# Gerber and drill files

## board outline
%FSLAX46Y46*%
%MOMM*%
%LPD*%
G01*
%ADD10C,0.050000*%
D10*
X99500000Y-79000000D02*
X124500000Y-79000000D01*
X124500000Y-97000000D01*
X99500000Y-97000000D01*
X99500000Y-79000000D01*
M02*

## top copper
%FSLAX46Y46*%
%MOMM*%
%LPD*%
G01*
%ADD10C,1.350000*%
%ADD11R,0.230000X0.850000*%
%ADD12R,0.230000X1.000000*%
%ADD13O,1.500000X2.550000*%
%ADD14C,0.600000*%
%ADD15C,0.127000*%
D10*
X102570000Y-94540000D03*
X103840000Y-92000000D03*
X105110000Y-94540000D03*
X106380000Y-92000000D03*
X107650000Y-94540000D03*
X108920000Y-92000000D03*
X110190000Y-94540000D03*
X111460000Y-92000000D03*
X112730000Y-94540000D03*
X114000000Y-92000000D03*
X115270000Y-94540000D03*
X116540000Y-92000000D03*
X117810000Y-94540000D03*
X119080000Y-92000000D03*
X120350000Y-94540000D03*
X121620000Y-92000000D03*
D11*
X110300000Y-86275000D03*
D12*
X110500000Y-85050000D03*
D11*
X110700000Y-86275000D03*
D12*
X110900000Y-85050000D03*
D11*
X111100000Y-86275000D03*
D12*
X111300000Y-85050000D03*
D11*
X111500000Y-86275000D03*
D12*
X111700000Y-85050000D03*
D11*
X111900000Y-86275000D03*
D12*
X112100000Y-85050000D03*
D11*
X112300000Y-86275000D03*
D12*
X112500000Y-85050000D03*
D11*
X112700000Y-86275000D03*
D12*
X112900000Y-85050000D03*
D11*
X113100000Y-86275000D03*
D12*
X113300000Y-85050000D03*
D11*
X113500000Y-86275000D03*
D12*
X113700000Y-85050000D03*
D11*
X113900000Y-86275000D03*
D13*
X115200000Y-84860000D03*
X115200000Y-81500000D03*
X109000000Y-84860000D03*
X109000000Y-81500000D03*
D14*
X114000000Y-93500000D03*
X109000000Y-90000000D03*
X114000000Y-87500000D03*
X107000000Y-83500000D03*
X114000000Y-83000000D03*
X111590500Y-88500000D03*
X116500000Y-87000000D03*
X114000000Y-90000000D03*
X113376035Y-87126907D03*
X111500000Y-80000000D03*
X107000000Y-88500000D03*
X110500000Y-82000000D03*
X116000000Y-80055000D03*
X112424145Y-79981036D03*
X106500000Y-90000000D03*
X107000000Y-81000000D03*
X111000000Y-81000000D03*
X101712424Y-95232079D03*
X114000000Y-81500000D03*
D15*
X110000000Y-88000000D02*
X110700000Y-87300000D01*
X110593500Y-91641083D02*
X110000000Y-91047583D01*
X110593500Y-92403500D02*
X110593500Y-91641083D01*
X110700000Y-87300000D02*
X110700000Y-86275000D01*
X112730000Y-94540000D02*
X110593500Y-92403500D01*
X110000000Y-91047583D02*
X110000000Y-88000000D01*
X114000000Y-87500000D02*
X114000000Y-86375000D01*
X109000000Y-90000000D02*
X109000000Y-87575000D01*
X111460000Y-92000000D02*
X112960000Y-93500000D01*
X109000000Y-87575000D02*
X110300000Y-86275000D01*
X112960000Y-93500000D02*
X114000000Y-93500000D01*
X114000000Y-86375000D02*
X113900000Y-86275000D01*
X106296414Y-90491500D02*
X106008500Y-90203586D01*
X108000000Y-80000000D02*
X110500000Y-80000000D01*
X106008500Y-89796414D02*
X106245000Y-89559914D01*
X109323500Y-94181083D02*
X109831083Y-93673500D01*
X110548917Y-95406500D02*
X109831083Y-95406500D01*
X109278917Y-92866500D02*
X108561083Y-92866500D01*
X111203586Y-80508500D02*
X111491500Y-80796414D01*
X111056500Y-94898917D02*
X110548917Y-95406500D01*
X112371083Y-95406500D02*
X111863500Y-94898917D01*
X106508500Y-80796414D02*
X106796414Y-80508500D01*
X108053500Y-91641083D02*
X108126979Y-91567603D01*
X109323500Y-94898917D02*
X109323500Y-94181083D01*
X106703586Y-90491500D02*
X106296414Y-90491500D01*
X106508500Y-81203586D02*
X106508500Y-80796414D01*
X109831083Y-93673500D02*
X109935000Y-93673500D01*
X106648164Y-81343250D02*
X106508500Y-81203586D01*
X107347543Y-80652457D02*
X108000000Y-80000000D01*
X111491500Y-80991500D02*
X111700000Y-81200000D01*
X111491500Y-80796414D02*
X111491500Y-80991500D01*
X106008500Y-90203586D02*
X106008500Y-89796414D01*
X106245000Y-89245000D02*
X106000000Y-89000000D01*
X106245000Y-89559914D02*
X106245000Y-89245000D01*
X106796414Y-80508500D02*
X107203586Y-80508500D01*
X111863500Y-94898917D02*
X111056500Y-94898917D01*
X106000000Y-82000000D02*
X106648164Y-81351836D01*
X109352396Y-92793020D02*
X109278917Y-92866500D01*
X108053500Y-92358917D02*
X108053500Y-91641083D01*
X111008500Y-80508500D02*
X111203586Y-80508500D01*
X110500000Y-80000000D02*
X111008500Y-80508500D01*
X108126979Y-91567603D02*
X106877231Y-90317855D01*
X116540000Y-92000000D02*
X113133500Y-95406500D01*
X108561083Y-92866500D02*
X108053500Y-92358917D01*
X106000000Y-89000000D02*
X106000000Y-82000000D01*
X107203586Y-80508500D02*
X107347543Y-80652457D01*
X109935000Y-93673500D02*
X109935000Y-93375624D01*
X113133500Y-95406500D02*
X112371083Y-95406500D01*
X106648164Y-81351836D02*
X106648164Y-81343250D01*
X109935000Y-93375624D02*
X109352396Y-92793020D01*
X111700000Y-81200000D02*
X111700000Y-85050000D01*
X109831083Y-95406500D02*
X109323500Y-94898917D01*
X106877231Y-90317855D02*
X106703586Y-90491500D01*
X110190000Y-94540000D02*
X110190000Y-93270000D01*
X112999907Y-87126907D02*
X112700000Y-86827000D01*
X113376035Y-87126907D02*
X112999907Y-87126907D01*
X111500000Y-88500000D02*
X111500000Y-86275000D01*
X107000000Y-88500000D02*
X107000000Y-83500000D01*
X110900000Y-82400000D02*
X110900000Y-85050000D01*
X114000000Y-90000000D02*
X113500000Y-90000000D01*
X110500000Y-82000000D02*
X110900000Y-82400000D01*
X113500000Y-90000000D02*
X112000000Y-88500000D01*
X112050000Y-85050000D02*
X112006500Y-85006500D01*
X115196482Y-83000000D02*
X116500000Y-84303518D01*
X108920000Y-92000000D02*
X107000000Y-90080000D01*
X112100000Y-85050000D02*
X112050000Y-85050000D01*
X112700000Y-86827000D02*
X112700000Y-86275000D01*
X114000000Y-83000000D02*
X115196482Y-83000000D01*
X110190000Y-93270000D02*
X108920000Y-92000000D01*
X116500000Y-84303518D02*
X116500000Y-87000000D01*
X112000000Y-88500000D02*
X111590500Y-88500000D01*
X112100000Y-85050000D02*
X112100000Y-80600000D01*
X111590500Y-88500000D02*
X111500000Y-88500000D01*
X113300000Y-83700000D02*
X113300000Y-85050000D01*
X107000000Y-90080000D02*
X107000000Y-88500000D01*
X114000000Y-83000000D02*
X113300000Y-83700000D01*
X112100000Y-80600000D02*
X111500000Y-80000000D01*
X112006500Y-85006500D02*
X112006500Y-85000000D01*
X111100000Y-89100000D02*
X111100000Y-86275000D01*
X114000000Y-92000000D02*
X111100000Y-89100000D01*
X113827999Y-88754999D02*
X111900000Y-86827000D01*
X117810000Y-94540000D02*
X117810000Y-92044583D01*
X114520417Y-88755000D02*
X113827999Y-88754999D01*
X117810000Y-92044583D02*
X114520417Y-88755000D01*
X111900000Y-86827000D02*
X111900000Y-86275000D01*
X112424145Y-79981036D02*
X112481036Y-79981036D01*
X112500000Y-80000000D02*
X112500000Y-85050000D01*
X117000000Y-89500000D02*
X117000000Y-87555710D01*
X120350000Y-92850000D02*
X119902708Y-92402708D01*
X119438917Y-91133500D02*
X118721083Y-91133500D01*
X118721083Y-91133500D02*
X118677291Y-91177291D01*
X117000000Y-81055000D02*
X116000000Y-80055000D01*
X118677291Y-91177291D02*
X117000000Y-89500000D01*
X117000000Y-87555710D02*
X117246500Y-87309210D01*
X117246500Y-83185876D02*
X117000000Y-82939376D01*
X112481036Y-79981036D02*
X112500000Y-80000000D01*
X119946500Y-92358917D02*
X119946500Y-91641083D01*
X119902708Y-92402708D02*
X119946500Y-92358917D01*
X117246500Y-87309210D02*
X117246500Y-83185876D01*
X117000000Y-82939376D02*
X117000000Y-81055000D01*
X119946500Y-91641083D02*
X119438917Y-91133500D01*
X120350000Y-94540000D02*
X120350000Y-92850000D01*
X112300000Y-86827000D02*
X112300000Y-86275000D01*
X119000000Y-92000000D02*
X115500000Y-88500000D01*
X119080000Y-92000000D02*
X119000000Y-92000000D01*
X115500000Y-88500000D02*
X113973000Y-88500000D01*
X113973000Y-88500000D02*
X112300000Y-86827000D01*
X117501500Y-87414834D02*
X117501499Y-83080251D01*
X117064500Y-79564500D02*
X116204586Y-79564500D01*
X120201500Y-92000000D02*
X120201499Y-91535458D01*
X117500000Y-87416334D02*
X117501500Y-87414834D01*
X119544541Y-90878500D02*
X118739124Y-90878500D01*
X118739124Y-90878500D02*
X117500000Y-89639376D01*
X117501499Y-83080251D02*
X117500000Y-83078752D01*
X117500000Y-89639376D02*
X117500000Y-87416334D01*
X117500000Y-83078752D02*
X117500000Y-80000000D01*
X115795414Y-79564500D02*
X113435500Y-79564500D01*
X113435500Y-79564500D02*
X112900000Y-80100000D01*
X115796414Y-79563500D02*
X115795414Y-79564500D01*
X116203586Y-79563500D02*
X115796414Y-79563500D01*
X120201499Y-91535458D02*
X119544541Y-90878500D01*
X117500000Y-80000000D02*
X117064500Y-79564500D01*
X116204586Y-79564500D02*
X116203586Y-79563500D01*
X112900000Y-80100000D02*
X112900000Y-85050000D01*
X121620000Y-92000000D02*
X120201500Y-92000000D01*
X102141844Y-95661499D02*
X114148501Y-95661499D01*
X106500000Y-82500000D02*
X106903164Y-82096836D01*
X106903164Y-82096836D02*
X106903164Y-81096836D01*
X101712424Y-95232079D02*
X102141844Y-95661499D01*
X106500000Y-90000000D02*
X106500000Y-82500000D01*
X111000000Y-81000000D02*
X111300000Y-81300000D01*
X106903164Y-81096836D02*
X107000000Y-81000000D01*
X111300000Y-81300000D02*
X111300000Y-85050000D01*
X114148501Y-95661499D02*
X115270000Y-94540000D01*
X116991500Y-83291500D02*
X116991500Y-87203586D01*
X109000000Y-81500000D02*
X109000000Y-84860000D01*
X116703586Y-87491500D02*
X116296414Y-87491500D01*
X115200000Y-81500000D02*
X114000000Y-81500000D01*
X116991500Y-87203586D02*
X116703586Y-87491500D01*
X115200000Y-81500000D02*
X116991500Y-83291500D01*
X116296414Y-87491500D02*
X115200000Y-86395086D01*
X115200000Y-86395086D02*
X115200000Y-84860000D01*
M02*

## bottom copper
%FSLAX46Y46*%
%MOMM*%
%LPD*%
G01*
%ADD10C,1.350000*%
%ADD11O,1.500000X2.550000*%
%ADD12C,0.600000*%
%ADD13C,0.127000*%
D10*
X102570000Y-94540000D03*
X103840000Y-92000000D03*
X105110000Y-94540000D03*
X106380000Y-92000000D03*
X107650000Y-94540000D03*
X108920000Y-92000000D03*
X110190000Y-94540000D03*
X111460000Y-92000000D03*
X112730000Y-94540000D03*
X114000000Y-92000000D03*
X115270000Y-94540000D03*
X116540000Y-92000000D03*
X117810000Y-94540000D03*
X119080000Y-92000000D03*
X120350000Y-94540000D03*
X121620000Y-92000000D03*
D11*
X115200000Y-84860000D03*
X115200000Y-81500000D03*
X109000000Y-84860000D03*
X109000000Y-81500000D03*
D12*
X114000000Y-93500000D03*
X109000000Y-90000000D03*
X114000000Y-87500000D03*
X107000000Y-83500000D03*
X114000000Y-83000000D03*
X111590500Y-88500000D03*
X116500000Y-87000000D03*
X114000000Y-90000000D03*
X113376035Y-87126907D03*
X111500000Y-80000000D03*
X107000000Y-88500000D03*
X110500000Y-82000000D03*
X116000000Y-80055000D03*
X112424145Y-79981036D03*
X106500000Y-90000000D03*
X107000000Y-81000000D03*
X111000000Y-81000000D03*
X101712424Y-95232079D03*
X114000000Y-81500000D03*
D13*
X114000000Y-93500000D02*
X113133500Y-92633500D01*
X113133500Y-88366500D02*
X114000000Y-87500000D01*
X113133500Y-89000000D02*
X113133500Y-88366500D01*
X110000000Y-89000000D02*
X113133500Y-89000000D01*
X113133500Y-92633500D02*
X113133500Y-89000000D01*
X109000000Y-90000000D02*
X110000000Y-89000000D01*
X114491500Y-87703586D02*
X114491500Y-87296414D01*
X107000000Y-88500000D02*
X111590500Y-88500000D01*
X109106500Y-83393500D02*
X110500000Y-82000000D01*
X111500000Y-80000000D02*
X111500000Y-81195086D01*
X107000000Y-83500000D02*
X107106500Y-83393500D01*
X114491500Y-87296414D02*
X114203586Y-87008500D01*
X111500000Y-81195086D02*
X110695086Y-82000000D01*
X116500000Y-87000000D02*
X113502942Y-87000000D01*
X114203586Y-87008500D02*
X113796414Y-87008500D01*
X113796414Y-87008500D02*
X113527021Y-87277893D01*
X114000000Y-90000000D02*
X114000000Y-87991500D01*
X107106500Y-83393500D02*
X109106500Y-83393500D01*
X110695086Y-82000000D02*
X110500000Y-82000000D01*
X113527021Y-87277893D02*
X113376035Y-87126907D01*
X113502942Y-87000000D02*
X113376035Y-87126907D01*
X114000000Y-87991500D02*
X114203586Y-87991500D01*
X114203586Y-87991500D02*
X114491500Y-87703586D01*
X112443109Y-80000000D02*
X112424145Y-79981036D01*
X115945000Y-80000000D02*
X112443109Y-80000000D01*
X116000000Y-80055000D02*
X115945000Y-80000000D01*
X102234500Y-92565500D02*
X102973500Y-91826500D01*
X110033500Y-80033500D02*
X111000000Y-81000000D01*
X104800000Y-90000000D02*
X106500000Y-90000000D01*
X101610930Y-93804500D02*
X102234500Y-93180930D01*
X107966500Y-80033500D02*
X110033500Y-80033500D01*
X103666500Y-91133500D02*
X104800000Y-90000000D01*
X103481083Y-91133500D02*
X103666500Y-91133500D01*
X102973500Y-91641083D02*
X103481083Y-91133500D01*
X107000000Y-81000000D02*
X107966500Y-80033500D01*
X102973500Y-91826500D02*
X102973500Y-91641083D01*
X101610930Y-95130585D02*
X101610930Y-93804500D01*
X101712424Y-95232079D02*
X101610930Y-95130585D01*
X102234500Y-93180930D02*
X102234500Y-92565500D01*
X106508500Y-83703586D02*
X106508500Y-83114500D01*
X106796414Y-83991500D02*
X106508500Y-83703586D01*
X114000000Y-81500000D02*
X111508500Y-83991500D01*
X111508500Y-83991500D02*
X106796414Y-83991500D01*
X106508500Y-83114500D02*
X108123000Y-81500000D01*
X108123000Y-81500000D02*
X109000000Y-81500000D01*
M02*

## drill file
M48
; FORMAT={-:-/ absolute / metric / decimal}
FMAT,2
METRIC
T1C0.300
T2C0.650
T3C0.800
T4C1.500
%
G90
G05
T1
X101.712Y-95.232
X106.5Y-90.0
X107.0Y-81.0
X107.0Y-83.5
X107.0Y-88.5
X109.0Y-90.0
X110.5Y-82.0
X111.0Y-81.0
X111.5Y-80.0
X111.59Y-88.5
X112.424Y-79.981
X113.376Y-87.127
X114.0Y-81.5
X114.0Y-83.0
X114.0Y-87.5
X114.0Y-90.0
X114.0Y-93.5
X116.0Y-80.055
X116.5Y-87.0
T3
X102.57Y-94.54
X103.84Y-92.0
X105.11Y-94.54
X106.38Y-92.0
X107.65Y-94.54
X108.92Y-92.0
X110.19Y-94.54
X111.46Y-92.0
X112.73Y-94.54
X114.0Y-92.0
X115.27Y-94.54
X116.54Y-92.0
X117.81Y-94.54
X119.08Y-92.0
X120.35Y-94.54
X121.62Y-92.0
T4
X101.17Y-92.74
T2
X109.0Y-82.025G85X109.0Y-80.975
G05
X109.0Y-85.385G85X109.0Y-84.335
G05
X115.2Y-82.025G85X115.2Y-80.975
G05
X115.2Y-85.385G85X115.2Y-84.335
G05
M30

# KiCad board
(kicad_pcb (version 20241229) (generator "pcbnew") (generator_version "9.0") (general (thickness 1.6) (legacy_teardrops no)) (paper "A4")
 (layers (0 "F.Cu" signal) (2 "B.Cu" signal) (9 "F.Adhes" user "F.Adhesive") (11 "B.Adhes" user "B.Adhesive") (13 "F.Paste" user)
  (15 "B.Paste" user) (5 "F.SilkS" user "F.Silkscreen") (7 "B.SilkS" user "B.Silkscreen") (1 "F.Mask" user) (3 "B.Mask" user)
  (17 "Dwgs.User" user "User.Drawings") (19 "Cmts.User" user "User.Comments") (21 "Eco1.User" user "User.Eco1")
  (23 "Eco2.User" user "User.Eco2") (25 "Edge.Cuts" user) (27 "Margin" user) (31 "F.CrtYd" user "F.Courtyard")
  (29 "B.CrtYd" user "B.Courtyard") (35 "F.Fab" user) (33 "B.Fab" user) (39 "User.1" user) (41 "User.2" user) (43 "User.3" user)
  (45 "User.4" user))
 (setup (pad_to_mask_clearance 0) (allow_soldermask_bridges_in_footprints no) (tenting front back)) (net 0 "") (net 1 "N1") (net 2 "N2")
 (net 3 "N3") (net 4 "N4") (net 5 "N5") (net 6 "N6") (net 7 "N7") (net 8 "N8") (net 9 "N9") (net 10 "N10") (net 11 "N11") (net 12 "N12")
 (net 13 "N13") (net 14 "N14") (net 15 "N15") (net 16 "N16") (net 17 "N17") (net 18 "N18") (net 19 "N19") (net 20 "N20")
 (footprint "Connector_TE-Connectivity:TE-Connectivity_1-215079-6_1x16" (layer "F.Cu") (at 111.46 93.27)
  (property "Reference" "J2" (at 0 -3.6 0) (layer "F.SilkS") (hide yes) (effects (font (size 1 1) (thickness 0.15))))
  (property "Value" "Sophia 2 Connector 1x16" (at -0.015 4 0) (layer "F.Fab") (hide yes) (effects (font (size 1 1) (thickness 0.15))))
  (pad "" np_thru_hole circle (at -10.29 -0.53) (size 1.5 1.5) (drill 1.5) (layers "*.Cu" "*.Mask"))
  (pad "1" thru_hole circle (at -8.89 1.27) (size 1.35 1.35) (drill 0.8) (layers "*.Cu" "*.Mask") (remove_unused_layers no) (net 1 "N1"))
  (pad "2" thru_hole circle (at -7.62 -1.27) (size 1.35 1.35) (drill 0.8) (layers "*.Cu" "*.Mask") (remove_unused_layers no) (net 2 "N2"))
  (pad "3" thru_hole circle (at -6.35 1.27) (size 1.35 1.35) (drill 0.8) (layers "*.Cu" "*.Mask") (remove_unused_layers no) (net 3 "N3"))
  (pad "4" thru_hole circle (at -5.08 -1.27) (size 1.35 1.35) (drill 0.8) (layers "*.Cu" "*.Mask") (remove_unused_layers no) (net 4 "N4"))
  (pad "5" thru_hole circle (at -3.81 1.27) (size 1.35 1.35) (drill 0.8) (layers "*.Cu" "*.Mask") (remove_unused_layers no) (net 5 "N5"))
  (pad "6" thru_hole circle (at -2.54 -1.27) (size 1.35 1.35) (drill 0.8) (layers "*.Cu" "*.Mask") (remove_unused_layers no) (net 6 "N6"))
  (pad "7" thru_hole circle (at -1.27 1.27) (size 1.35 1.35) (drill 0.8) (layers "*.Cu" "*.Mask") (remove_unused_layers no) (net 6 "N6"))
  (pad "8" thru_hole circle (at 0 -1.27) (size 1.35 1.35) (drill 0.8) (layers "*.Cu" "*.Mask") (remove_unused_layers no) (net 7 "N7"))
  (pad "9" thru_hole circle (at 1.27 1.27) (size 1.35 1.35) (drill 0.8) (layers "*.Cu" "*.Mask") (remove_unused_layers no) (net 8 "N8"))
  (pad "10" thru_hole circle (at 2.54 -1.27) (size 1.35 1.35) (drill 0.8) (layers "*.Cu" "*.Mask") (remove_unused_layers no) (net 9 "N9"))
  (pad "11" thru_hole circle (at 3.81 1.27) (size 1.35 1.35) (drill 0.8) (layers "*.Cu" "*.Mask") (remove_unused_layers no) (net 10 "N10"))
  (pad "12" thru_hole circle (at 5.08 -1.27) (size 1.35 1.35) (drill 0.8) (layers "*.Cu" "*.Mask") (remove_unused_layers no) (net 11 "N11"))
  (pad "13" thru_hole circle (at 6.35 1.27) (size 1.35 1.35) (drill 0.8) (layers "*.Cu" "*.Mask") (remove_unused_layers no) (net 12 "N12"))
  (pad "14" thru_hole circle (at 7.62 -1.27) (size 1.35 1.35) (drill 0.8) (layers "*.Cu" "*.Mask") (remove_unused_layers no) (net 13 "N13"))
  (pad "15" thru_hole circle (at 8.89 1.27) (size 1.35 1.35) (drill 0.8) (layers "*.Cu" "*.Mask") (remove_unused_layers no) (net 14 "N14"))
  (pad "16" thru_hole circle (at 10.16 -1.27) (size 1.35 1.35) (drill 0.8) (layers "*.Cu" "*.Mask") (remove_unused_layers no) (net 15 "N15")))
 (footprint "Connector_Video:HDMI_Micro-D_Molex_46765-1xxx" (layer "F.Cu") (at 112.1 81.5 180)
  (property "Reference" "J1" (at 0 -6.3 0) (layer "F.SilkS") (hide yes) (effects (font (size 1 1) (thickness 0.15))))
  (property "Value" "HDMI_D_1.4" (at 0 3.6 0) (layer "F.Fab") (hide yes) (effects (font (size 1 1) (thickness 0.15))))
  (pad "1" smd rect (at 1.8 -4.775 180) (size 0.23 0.85) (layers "F.Cu" "F.Mask" "F.Paste") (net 7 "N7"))
  (pad "2" smd rect (at 1.6 -3.55 180) (size 0.23 1) (layers "F.Cu" "F.Mask" "F.Paste") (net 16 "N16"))
  (pad "3" smd rect (at 1.4 -4.775 180) (size 0.23 0.85) (layers "F.Cu" "F.Mask" "F.Paste") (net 8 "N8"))
  (pad "4" smd rect (at 1.2 -3.55 180) (size 0.23 1) (layers "F.Cu" "F.Mask" "F.Paste") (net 6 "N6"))
  (pad "5" smd rect (at 1 -4.775 180) (size 0.23 0.85) (layers "F.Cu" "F.Mask" "F.Paste") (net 9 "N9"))
  (pad "6" smd rect (at 0.8 -3.55 180) (size 0.23 1) (layers "F.Cu" "F.Mask" "F.Paste") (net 10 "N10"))
  (pad "7" smd rect (at 0.6 -4.775 180) (size 0.23 0.85) (layers "F.Cu" "F.Mask" "F.Paste") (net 6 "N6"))
  (pad "8" smd rect (at 0.4 -3.55 180) (size 0.23 1) (layers "F.Cu" "F.Mask" "F.Paste") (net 11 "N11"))
  (pad "9" smd rect (at 0.2 -4.775 180) (size 0.23 0.85) (layers "F.Cu" "F.Mask" "F.Paste") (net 12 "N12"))
  (pad "10" smd rect (at 0 -3.55 180) (size 0.23 1) (layers "F.Cu" "F.Mask" "F.Paste") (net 6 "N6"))
  (pad "11" smd rect (at -0.2 -4.775 180) (size 0.23 0.85) (layers "F.Cu" "F.Mask" "F.Paste") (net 13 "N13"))
  (pad "12" smd rect (at -0.4 -3.55 180) (size 0.23 1) (layers "F.Cu" "F.Mask" "F.Paste") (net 14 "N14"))
  (pad "13" smd rect (at -0.6 -4.775 180) (size 0.23 0.85) (layers "F.Cu" "F.Mask" "F.Paste") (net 6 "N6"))
  (pad "14" smd rect (at -0.8 -3.55 180) (size 0.23 1) (layers "F.Cu" "F.Mask" "F.Paste") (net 15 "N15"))
  (pad "15" smd rect (at -1 -4.775 180) (size 0.23 0.85) (layers "F.Cu" "F.Mask" "F.Paste") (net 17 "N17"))
  (pad "16" smd rect (at -1.2 -3.55 180) (size 0.23 1) (layers "F.Cu" "F.Mask" "F.Paste") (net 6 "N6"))
  (pad "17" smd rect (at -1.4 -4.775 180) (size 0.23 0.85) (layers "F.Cu" "F.Mask" "F.Paste") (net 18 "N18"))
  (pad "18" smd rect (at -1.6 -3.55 180) (size 0.23 1) (layers "F.Cu" "F.Mask" "F.Paste") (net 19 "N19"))
  (pad "19" smd rect (at -1.8 -4.775 180) (size 0.23 0.85) (layers "F.Cu" "F.Mask" "F.Paste") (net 7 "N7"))
  (pad "SH" thru_hole oval (at -3.1 -3.36 180) (size 1.5 2.55) (drill oval 0.65 1.7) (layers "*.Cu" "*.Mask") (remove_unused_layers no)
   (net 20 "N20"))
  (pad "SH" thru_hole oval (at -3.1 0 180) (size 1.5 2.55) (drill oval 0.65 1.7) (layers "*.Cu" "*.Mask") (remove_unused_layers no)
   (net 20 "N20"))
  (pad "SH" thru_hole oval (at 3.1 -3.36 180) (size 1.5 2.55) (drill oval 0.65 1.7) (layers "*.Cu" "*.Mask") (remove_unused_layers no)
   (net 20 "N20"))
  (pad "SH" thru_hole oval (at 3.1 0 180) (size 1.5 2.55) (drill oval 0.65 1.7) (layers "*.Cu" "*.Mask") (remove_unused_layers no)
   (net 20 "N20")))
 (gr_rect (start 99.5 79) (end 124.5 97) (stroke (width 0.05) (type default)) (fill no) (layer "Edge.Cuts"))
 (segment (start 110 88) (end 110.7 87.3) (width 0.127) (layer "F.Cu") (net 8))
 (segment (start 110.5935 91.641083) (end 110 91.047583) (width 0.127) (layer "F.Cu") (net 8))
 (segment (start 110.5935 92.4035) (end 110.5935 91.641083) (width 0.127) (layer "F.Cu") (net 8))
 (segment (start 110.7 87.3) (end 110.7 86.275) (width 0.127) (layer "F.Cu") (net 8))
 (segment (start 112.73 94.54) (end 110.5935 92.4035) (width 0.127) (layer "F.Cu") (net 8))
 (segment (start 110 91.047583) (end 110 88) (width 0.127) (layer "F.Cu") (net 8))
 (segment (start 114 87.5) (end 114 86.375) (width 0.127) (layer "F.Cu") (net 7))
 (segment (start 109 90) (end 109 87.575) (width 0.127) (layer "F.Cu") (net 7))
 (segment (start 111.46 92) (end 112.96 93.5) (width 0.127) (layer "F.Cu") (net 7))
 (segment (start 109 87.575) (end 110.3 86.275) (width 0.127) (layer "F.Cu") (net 7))
 (segment (start 112.96 93.5) (end 114 93.5) (width 0.127) (layer "F.Cu") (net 7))
 (segment (start 114 86.375) (end 113.9 86.275) (width 0.127) (layer "F.Cu") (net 7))
 (via (at 114 93.5) (size 0.6) (drill 0.3) (layers "F.Cu" "B.Cu") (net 7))
 (via (at 109 90) (size 0.6) (drill 0.3) (layers "F.Cu" "B.Cu") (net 7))
 (via (at 114 87.5) (size 0.6) (drill 0.3) (layers "F.Cu" "B.Cu") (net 7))
 (segment (start 114 93.5) (end 113.1335 92.6335) (width 0.127) (layer "B.Cu") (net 7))
 (segment (start 113.1335 88.3665) (end 114 87.5) (width 0.127) (layer "B.Cu") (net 7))
 (segment (start 113.1335 89) (end 113.1335 88.3665) (width 0.127) (layer "B.Cu") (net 7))
 (segment (start 110 89) (end 113.1335 89) (width 0.127) (layer "B.Cu") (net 7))
 (segment (start 113.1335 92.6335) (end 113.1335 89) (width 0.127) (layer "B.Cu") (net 7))
 (segment (start 109 90) (end 110 89) (width 0.127) (layer "B.Cu") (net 7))
 (segment (start 106.296414 90.4915) (end 106.0085 90.203586) (width 0.127) (layer "F.Cu") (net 11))
 (segment (start 108 80) (end 110.5 80) (width 0.127) (layer "F.Cu") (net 11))
 (segment (start 106.0085 89.796414) (end 106.245 89.559914) (width 0.127) (layer "F.Cu") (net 11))
 (segment (start 109.3235 94.181083) (end 109.831083 93.6735) (width 0.127) (layer "F.Cu") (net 11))
 (segment (start 110.548917 95.4065) (end 109.831083 95.4065) (width 0.127) (layer "F.Cu") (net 11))
 (segment (start 109.278917 92.8665) (end 108.561083 92.8665) (width 0.127) (layer "F.Cu") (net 11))
 (segment (start 111.203586 80.5085) (end 111.4915 80.796414) (width 0.127) (layer "F.Cu") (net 11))
 (segment (start 111.0565 94.898917) (end 110.548917 95.4065) (width 0.127) (layer "F.Cu") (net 11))
 (segment (start 112.371083 95.4065) (end 111.8635 94.898917) (width 0.127) (layer "F.Cu") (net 11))
 (segment (start 106.5085 80.796414) (end 106.796414 80.5085) (width 0.127) (layer "F.Cu") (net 11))
 (segment (start 108.0535 91.641083) (end 108.126979 91.567603) (width 0.127) (layer "F.Cu") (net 11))
 (segment (start 109.3235 94.898917) (end 109.3235 94.181083) (width 0.127) (layer "F.Cu") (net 11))
 (segment (start 106.703586 90.4915) (end 106.296414 90.4915) (width 0.127) (layer "F.Cu") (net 11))
 (segment (start 106.5085 81.203586) (end 106.5085 80.796414) (width 0.127) (layer "F.Cu") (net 11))
 (segment (start 109.831083 93.6735) (end 109.935 93.6735) (width 0.127) (layer "F.Cu") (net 11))
 (segment (start 106.648164 81.34325) (end 106.5085 81.203586) (width 0.127) (layer "F.Cu") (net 11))
 (segment (start 107.347543 80.652457) (end 108 80) (width 0.127) (layer "F.Cu") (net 11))
 (segment (start 111.4915 80.9915) (end 111.7 81.2) (width 0.127) (layer "F.Cu") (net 11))
 (segment (start 111.4915 80.796414) (end 111.4915 80.9915) (width 0.127) (layer "F.Cu") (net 11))
 (segment (start 106.0085 90.203586) (end 106.0085 89.796414) (width 0.127) (layer "F.Cu") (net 11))
 (segment (start 106.245 89.245) (end 106 89) (width 0.127) (layer "F.Cu") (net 11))
 (segment (start 106.245 89.559914) (end 106.245 89.245) (width 0.127) (layer "F.Cu") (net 11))
 (segment (start 106.796414 80.5085) (end 107.203586 80.5085) (width 0.127) (layer "F.Cu") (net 11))
 (segment (start 111.8635 94.898917) (end 111.0565 94.898917) (width 0.127) (layer "F.Cu") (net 11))
 (segment (start 106 82) (end 106.648164 81.351836) (width 0.127) (layer "F.Cu") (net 11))
 (segment (start 109.352396 92.79302) (end 109.278917 92.8665) (width 0.127) (layer "F.Cu") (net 11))
 (segment (start 108.0535 92.358917) (end 108.0535 91.641083) (width 0.127) (layer "F.Cu") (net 11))
 (segment (start 111.0085 80.5085) (end 111.203586 80.5085) (width 0.127) (layer "F.Cu") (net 11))
 (segment (start 110.5 80) (end 111.0085 80.5085) (width 0.127) (layer "F.Cu") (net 11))
 (segment (start 108.126979 91.567603) (end 106.877231 90.317855) (width 0.127) (layer "F.Cu") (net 11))
 (segment (start 116.54 92) (end 113.1335 95.4065) (width 0.127) (layer "F.Cu") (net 11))
 (segment (start 108.561083 92.8665) (end 108.0535 92.358917) (width 0.127) (layer "F.Cu") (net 11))
 (segment (start 106 89) (end 106 82) (width 0.127) (layer "F.Cu") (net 11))
 (segment (start 107.203586 80.5085) (end 107.347543 80.652457) (width 0.127) (layer "F.Cu") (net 11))
 (segment (start 109.935 93.6735) (end 109.935 93.375624) (width 0.127) (layer "F.Cu") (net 11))
 (segment (start 113.1335 95.4065) (end 112.371083 95.4065) (width 0.127) (layer "F.Cu") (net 11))
 (segment (start 106.648164 81.351836) (end 106.648164 81.34325) (width 0.127) (layer "F.Cu") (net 11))
 (segment (start 109.935 93.375624) (end 109.352396 92.79302) (width 0.127) (layer "F.Cu") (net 11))
 (segment (start 111.7 81.2) (end 111.7 85.05) (width 0.127) (layer "F.Cu") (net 11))
 (segment (start 109.831083 95.4065) (end 109.3235 94.898917) (width 0.127) (layer "F.Cu") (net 11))
 (segment (start 106.877231 90.317855) (end 106.703586 90.4915) (width 0.127) (layer "F.Cu") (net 11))
 (segment (start 110.19 94.54) (end 110.19 93.27) (width 0.127) (layer "F.Cu") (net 6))
 (segment (start 112.999907 87.126907) (end 112.7 86.827) (width 0.127) (layer "F.Cu") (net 6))
 (segment (start 113.376035 87.126907) (end 112.999907 87.126907) (width 0.127) (layer "F.Cu") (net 6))
 (segment (start 111.5 88.5) (end 111.5 86.275) (width 0.127) (layer "F.Cu") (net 6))
 (segment (start 107 88.5) (end 107 83.5) (width 0.127) (layer "F.Cu") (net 6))
 (segment (start 110.9 82.4) (end 110.9 85.05) (width 0.127) (layer "F.Cu") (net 6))
 (segment (start 114 90) (end 113.5 90) (width 0.127) (layer "F.Cu") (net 6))
 (segment (start 110.5 82) (end 110.9 82.4) (width 0.127) (layer "F.Cu") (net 6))
 (segment (start 113.5 90) (end 112 88.5) (width 0.127) (layer "F.Cu") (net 6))
 (segment (start 112.05 85.05) (end 112.0065 85.0065) (width 0.127) (layer "F.Cu") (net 6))
 (segment (start 115.196482 83) (end 116.5 84.303518) (width 0.127) (layer "F.Cu") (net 6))
 (segment (start 108.92 92) (end 107 90.08) (width 0.127) (layer "F.Cu") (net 6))
 (segment (start 112.1 85.05) (end 112.05 85.05) (width 0.127) (layer "F.Cu") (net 6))
 (segment (start 112.7 86.827) (end 112.7 86.275) (width 0.127) (layer "F.Cu") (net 6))
 (segment (start 114 83) (end 115.196482 83) (width 0.127) (layer "F.Cu") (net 6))
 (segment (start 110.19 93.27) (end 108.92 92) (width 0.127) (layer "F.Cu") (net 6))
 (segment (start 116.5 84.303518) (end 116.5 87) (width 0.127) (layer "F.Cu") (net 6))
 (segment (start 112 88.5) (end 111.5905 88.5) (width 0.127) (layer "F.Cu") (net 6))
 (segment (start 112.1 85.05) (end 112.1 80.6) (width 0.127) (layer "F.Cu") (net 6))
 (segment (start 111.5905 88.5) (end 111.5 88.5) (width 0.127) (layer "F.Cu") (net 6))
 (segment (start 113.3 83.7) (end 113.3 85.05) (width 0.127) (layer "F.Cu") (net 6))
 (segment (start 107 90.08) (end 107 88.5) (width 0.127) (layer "F.Cu") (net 6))
 (segment (start 114 83) (end 113.3 83.7) (width 0.127) (layer "F.Cu") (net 6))
 (segment (start 112.1 80.6) (end 111.5 80) (width 0.127) (layer "F.Cu") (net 6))
 (segment (start 112.0065 85.0065) (end 112.0065 85) (width 0.127) (layer "F.Cu") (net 6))
 (via (at 107 83.5) (size 0.6) (drill 0.3) (layers "F.Cu" "B.Cu") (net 6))
 (via (at 114 83) (size 0.6) (drill 0.3) (layers "F.Cu" "B.Cu") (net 6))
 (via (at 111.5905 88.5) (size 0.6) (drill 0.3) (layers "F.Cu" "B.Cu") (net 6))
 (via (at 116.5 87) (size 0.6) (drill 0.3) (layers "F.Cu" "B.Cu") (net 6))
 (via (at 114 90) (size 0.6) (drill 0.3) (layers "F.Cu" "B.Cu") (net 6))
 (via (at 113.376035 87.126907) (size 0.6) (drill 0.3) (layers "F.Cu" "B.Cu") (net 6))
 (via (at 111.5 80) (size 0.6) (drill 0.3) (layers "F.Cu" "B.Cu") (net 6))
 (via (at 107 88.5) (size 0.6) (drill 0.3) (layers "F.Cu" "B.Cu") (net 6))
 (via (at 110.5 82) (size 0.6) (drill 0.3) (layers "F.Cu" "B.Cu") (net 6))
 (segment (start 114.4915 87.703586) (end 114.4915 87.296414) (width 0.127) (layer "B.Cu") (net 6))
 (segment (start 107 88.5) (end 111.5905 88.5) (width 0.127) (layer "B.Cu") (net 6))
 (segment (start 109.1065 83.3935) (end 110.5 82) (width 0.127) (layer "B.Cu") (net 6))
 (segment (start 111.5 80) (end 111.5 81.195086) (width 0.127) (layer "B.Cu") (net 6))
 (segment (start 107 83.5) (end 107.1065 83.3935) (width 0.127) (layer "B.Cu") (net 6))
 (segment (start 114.4915 87.296414) (end 114.203586 87.0085) (width 0.127) (layer "B.Cu") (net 6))
 (segment (start 111.5 81.195086) (end 110.695086 82) (width 0.127) (layer "B.Cu") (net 6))
 (segment (start 116.5 87) (end 113.502942 87) (width 0.127) (layer "B.Cu") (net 6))
 (segment (start 114.203586 87.0085) (end 113.796414 87.0085) (width 0.127) (layer "B.Cu") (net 6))
 (segment (start 113.796414 87.0085) (end 113.527021 87.277893) (width 0.127) (layer "B.Cu") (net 6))
 (segment (start 114 90) (end 114 87.9915) (width 0.127) (layer "B.Cu") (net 6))
 (segment (start 107.1065 83.3935) (end 109.1065 83.3935) (width 0.127) (layer "B.Cu") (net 6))
 (segment (start 110.695086 82) (end 110.5 82) (width 0.127) (layer "B.Cu") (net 6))
 (segment (start 113.527021 87.277893) (end 113.376035 87.126907) (width 0.127) (layer "B.Cu") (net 6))
 (segment (start 113.502942 87) (end 113.376035 87.126907) (width 0.127) (layer "B.Cu") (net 6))
 (segment (start 114 87.9915) (end 114.203586 87.9915) (width 0.127) (layer "B.Cu") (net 6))
 (segment (start 114.203586 87.9915) (end 114.4915 87.703586) (width 0.127) (layer "B.Cu") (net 6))
 (segment (start 111.1 89.1) (end 111.1 86.275) (width 0.127) (layer "F.Cu") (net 9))
 (segment (start 114 92) (end 111.1 89.1) (width 0.127) (layer "F.Cu") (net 9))
 (segment (start 113.827999 88.754999) (end 111.9 86.827) (width 0.127) (layer "F.Cu") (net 12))
 (segment (start 117.81 94.54) (end 117.81 92.044583) (width 0.127) (layer "F.Cu") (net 12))
 (segment (start 114.520417 88.755) (end 113.827999 88.754999) (width 0.127) (layer "F.Cu") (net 12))
 (segment (start 117.81 92.044583) (end 114.520417 88.755) (width 0.127) (layer "F.Cu") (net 12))
 (segment (start 111.9 86.827) (end 111.9 86.275) (width 0.127) (layer "F.Cu") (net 12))
 (segment (start 112.424145 79.981036) (end 112.481036 79.981036) (width 0.127) (layer "F.Cu") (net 14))
 (segment (start 112.5 80) (end 112.5 85.05) (width 0.127) (layer "F.Cu") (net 14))
 (segment (start 117 89.5) (end 117 87.55571) (width 0.127) (layer "F.Cu") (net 14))
 (segment (start 120.35 92.85) (end 119.902708 92.402708) (width 0.127) (layer "F.Cu") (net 14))
 (segment (start 119.438917 91.1335) (end 118.721083 91.1335) (width 0.127) (layer "F.Cu") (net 14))
 (segment (start 118.721083 91.1335) (end 118.677291 91.177291) (width 0.127) (layer "F.Cu") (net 14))
 (segment (start 117 81.055) (end 116 80.055) (width 0.127) (layer "F.Cu") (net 14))
 (segment (start 118.677291 91.177291) (end 117 89.5) (width 0.127) (layer "F.Cu") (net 14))
 (segment (start 117 87.55571) (end 117.2465 87.30921) (width 0.127) (layer "F.Cu") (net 14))
 (segment (start 117.2465 83.185876) (end 117 82.939376) (width 0.127) (layer "F.Cu") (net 14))
 (segment (start 112.481036 79.981036) (end 112.5 80) (width 0.127) (layer "F.Cu") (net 14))
 (segment (start 119.9465 92.358917) (end 119.9465 91.641083) (width 0.127) (layer "F.Cu") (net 14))
 (segment (start 119.902708 92.402708) (end 119.9465 92.358917) (width 0.127) (layer "F.Cu") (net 14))
 (segment (start 117.2465 87.30921) (end 117.2465 83.185876) (width 0.127) (layer "F.Cu") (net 14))
 (segment (start 117 82.939376) (end 117 81.055) (width 0.127) (layer "F.Cu") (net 14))
 (segment (start 119.9465 91.641083) (end 119.438917 91.1335) (width 0.127) (layer "F.Cu") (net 14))
 (segment (start 120.35 94.54) (end 120.35 92.85) (width 0.127) (layer "F.Cu") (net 14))
 (via (at 116 80.055) (size 0.6) (drill 0.3) (layers "F.Cu" "B.Cu") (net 14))
 (via (at 112.424145 79.981036) (size 0.6) (drill 0.3) (layers "F.Cu" "B.Cu") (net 14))
 (segment (start 112.443109 80) (end 112.424145 79.981036) (width 0.127) (layer "B.Cu") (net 14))
 (segment (start 115.945 80) (end 112.443109 80) (width 0.127) (layer "B.Cu") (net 14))
 (segment (start 116 80.055) (end 115.945 80) (width 0.127) (layer "B.Cu") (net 14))
 (segment (start 112.3 86.827) (end 112.3 86.275) (width 0.127) (layer "F.Cu") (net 13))
 (segment (start 119 92) (end 115.5 88.5) (width 0.127) (layer "F.Cu") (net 13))
 (segment (start 119.08 92) (end 119 92) (width 0.127) (layer "F.Cu") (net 13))
 (segment (start 115.5 88.5) (end 113.973 88.5) (width 0.127) (layer "F.Cu") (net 13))
 (segment (start 113.973 88.5) (end 112.3 86.827) (width 0.127) (layer "F.Cu") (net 13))
 (segment (start 117.5015 87.414834) (end 117.501499 83.080251) (width 0.127) (layer "F.Cu") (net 15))
 (segment (start 117.0645 79.5645) (end 116.204586 79.5645) (width 0.127) (layer "F.Cu") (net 15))
 (segment (start 120.2015 92) (end 120.201499 91.535458) (width 0.127) (layer "F.Cu") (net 15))
 (segment (start 117.5 87.416334) (end 117.5015 87.414834) (width 0.127) (layer "F.Cu") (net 15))
 (segment (start 119.544541 90.8785) (end 118.739124 90.8785) (width 0.127) (layer "F.Cu") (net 15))
 (segment (start 118.739124 90.8785) (end 117.5 89.639376) (width 0.127) (layer "F.Cu") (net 15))
 (segment (start 117.501499 83.080251) (end 117.5 83.078752) (width 0.127) (layer "F.Cu") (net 15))
 (segment (start 117.5 89.639376) (end 117.5 87.416334) (width 0.127) (layer "F.Cu") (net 15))
 (segment (start 117.5 83.078752) (end 117.5 80) (width 0.127) (layer "F.Cu") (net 15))
 (segment (start 115.795414 79.5645) (end 113.4355 79.5645) (width 0.127) (layer "F.Cu") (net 15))
 (segment (start 113.4355 79.5645) (end 112.9 80.1) (width 0.127) (layer "F.Cu") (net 15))
 (segment (start 115.796414 79.5635) (end 115.795414 79.5645) (width 0.127) (layer "F.Cu") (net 15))
 (segment (start 116.203586 79.5635) (end 115.796414 79.5635) (width 0.127) (layer "F.Cu") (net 15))
 (segment (start 120.201499 91.535458) (end 119.544541 90.8785) (width 0.127) (layer "F.Cu") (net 15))
 (segment (start 117.5 80) (end 117.0645 79.5645) (width 0.127) (layer "F.Cu") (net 15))
 (segment (start 116.204586 79.5645) (end 116.203586 79.5635) (width 0.127) (layer "F.Cu") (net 15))
 (segment (start 112.9 80.1) (end 112.9 85.05) (width 0.127) (layer "F.Cu") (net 15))
 (segment (start 121.62 92) (end 120.2015 92) (width 0.127) (layer "F.Cu") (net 15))
 (segment (start 102.141844 95.661499) (end 114.148501 95.661499) (width 0.127) (layer "F.Cu") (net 10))
 (segment (start 106.5 82.5) (end 106.903164 82.096836) (width 0.127) (layer "F.Cu") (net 10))
 (segment (start 106.903164 82.096836) (end 106.903164 81.096836) (width 0.127) (layer "F.Cu") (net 10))
 (segment (start 101.712424 95.232079) (end 102.141844 95.661499) (width 0.127) (layer "F.Cu") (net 10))
 (segment (start 106.5 90) (end 106.5 82.5) (width 0.127) (layer "F.Cu") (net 10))
 (segment (start 111 81) (end 111.3 81.3) (width 0.127) (layer "F.Cu") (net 10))
 (segment (start 106.903164 81.096836) (end 107 81) (width 0.127) (layer "F.Cu") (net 10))
 (segment (start 111.3 81.3) (end 111.3 85.05) (width 0.127) (layer "F.Cu") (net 10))
 (segment (start 114.148501 95.661499) (end 115.27 94.54) (width 0.127) (layer "F.Cu") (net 10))
 (via (at 106.5 90) (size 0.6) (drill 0.3) (layers "F.Cu" "B.Cu") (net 10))
 (via (at 107 81) (size 0.6) (drill 0.3) (layers "F.Cu" "B.Cu") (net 10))
 (via (at 111 81) (size 0.6) (drill 0.3) (layers "F.Cu" "B.Cu") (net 10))
 (via (at 101.712424 95.232079) (size 0.6) (drill 0.3) (layers "F.Cu" "B.Cu") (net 10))
 (segment (start 102.2345 92.5655) (end 102.9735 91.8265) (width 0.127) (layer "B.Cu") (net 10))
 (segment (start 110.0335 80.0335) (end 111 81) (width 0.127) (layer "B.Cu") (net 10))
 (segment (start 104.8 90) (end 106.5 90) (width 0.127) (layer "B.Cu") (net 10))
 (segment (start 101.61093 93.8045) (end 102.2345 93.18093) (width 0.127) (layer "B.Cu") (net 10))
 (segment (start 107.9665 80.0335) (end 110.0335 80.0335) (width 0.127) (layer "B.Cu") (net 10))
 (segment (start 103.6665 91.1335) (end 104.8 90) (width 0.127) (layer "B.Cu") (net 10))
 (segment (start 103.481083 91.1335) (end 103.6665 91.1335) (width 0.127) (layer "B.Cu") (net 10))
 (segment (start 102.9735 91.641083) (end 103.481083 91.1335) (width 0.127) (layer "B.Cu") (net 10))
 (segment (start 107 81) (end 107.9665 80.0335) (width 0.127) (layer "B.Cu") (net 10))
 (segment (start 102.9735 91.8265) (end 102.9735 91.641083) (width 0.127) (layer "B.Cu") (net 10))
 (segment (start 101.61093 95.130585) (end 101.61093 93.8045) (width 0.127) (layer "B.Cu") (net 10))
 (segment (start 101.712424 95.232079) (end 101.61093 95.130585) (width 0.127) (layer "B.Cu") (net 10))
 (segment (start 102.2345 93.18093) (end 102.2345 92.5655) (width 0.127) (layer "B.Cu") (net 10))
 (segment (start 116.9915 83.2915) (end 116.9915 87.203586) (width 0.127) (layer "F.Cu") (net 20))
 (segment (start 109 81.5) (end 109 84.86) (width 0.127) (layer "F.Cu") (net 20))
 (segment (start 116.703586 87.4915) (end 116.296414 87.4915) (width 0.127) (layer "F.Cu") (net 20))
 (segment (start 115.2 81.5) (end 114 81.5) (width 0.127) (layer "F.Cu") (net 20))
 (segment (start 116.9915 87.203586) (end 116.703586 87.4915) (width 0.127) (layer "F.Cu") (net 20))
 (segment (start 115.2 81.5) (end 116.9915 83.2915) (width 0.127) (layer "F.Cu") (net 20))
 (segment (start 116.296414 87.4915) (end 115.2 86.395086) (width 0.127) (layer "F.Cu") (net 20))
 (segment (start 115.2 86.395086) (end 115.2 84.86) (width 0.127) (layer "F.Cu") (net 20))
 (via (at 114 81.5) (size 0.6) (drill 0.3) (layers "F.Cu" "B.Cu") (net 20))
 (segment (start 106.5085 83.703586) (end 106.5085 83.1145) (width 0.127) (layer "B.Cu") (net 20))
 (segment (start 106.796414 83.9915) (end 106.5085 83.703586) (width 0.127) (layer "B.Cu") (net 20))
 (segment (start 114 81.5) (end 111.5085 83.9915) (width 0.127) (layer "B.Cu") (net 20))
 (segment (start 111.5085 83.9915) (end 106.796414 83.9915) (width 0.127) (layer "B.Cu") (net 20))
 (segment (start 106.5085 83.1145) (end 108.123 81.5) (width 0.127) (layer "B.Cu") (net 20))
 (segment (start 108.123 81.5) (end 109 81.5) (width 0.127) (layer "B.Cu") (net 20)))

